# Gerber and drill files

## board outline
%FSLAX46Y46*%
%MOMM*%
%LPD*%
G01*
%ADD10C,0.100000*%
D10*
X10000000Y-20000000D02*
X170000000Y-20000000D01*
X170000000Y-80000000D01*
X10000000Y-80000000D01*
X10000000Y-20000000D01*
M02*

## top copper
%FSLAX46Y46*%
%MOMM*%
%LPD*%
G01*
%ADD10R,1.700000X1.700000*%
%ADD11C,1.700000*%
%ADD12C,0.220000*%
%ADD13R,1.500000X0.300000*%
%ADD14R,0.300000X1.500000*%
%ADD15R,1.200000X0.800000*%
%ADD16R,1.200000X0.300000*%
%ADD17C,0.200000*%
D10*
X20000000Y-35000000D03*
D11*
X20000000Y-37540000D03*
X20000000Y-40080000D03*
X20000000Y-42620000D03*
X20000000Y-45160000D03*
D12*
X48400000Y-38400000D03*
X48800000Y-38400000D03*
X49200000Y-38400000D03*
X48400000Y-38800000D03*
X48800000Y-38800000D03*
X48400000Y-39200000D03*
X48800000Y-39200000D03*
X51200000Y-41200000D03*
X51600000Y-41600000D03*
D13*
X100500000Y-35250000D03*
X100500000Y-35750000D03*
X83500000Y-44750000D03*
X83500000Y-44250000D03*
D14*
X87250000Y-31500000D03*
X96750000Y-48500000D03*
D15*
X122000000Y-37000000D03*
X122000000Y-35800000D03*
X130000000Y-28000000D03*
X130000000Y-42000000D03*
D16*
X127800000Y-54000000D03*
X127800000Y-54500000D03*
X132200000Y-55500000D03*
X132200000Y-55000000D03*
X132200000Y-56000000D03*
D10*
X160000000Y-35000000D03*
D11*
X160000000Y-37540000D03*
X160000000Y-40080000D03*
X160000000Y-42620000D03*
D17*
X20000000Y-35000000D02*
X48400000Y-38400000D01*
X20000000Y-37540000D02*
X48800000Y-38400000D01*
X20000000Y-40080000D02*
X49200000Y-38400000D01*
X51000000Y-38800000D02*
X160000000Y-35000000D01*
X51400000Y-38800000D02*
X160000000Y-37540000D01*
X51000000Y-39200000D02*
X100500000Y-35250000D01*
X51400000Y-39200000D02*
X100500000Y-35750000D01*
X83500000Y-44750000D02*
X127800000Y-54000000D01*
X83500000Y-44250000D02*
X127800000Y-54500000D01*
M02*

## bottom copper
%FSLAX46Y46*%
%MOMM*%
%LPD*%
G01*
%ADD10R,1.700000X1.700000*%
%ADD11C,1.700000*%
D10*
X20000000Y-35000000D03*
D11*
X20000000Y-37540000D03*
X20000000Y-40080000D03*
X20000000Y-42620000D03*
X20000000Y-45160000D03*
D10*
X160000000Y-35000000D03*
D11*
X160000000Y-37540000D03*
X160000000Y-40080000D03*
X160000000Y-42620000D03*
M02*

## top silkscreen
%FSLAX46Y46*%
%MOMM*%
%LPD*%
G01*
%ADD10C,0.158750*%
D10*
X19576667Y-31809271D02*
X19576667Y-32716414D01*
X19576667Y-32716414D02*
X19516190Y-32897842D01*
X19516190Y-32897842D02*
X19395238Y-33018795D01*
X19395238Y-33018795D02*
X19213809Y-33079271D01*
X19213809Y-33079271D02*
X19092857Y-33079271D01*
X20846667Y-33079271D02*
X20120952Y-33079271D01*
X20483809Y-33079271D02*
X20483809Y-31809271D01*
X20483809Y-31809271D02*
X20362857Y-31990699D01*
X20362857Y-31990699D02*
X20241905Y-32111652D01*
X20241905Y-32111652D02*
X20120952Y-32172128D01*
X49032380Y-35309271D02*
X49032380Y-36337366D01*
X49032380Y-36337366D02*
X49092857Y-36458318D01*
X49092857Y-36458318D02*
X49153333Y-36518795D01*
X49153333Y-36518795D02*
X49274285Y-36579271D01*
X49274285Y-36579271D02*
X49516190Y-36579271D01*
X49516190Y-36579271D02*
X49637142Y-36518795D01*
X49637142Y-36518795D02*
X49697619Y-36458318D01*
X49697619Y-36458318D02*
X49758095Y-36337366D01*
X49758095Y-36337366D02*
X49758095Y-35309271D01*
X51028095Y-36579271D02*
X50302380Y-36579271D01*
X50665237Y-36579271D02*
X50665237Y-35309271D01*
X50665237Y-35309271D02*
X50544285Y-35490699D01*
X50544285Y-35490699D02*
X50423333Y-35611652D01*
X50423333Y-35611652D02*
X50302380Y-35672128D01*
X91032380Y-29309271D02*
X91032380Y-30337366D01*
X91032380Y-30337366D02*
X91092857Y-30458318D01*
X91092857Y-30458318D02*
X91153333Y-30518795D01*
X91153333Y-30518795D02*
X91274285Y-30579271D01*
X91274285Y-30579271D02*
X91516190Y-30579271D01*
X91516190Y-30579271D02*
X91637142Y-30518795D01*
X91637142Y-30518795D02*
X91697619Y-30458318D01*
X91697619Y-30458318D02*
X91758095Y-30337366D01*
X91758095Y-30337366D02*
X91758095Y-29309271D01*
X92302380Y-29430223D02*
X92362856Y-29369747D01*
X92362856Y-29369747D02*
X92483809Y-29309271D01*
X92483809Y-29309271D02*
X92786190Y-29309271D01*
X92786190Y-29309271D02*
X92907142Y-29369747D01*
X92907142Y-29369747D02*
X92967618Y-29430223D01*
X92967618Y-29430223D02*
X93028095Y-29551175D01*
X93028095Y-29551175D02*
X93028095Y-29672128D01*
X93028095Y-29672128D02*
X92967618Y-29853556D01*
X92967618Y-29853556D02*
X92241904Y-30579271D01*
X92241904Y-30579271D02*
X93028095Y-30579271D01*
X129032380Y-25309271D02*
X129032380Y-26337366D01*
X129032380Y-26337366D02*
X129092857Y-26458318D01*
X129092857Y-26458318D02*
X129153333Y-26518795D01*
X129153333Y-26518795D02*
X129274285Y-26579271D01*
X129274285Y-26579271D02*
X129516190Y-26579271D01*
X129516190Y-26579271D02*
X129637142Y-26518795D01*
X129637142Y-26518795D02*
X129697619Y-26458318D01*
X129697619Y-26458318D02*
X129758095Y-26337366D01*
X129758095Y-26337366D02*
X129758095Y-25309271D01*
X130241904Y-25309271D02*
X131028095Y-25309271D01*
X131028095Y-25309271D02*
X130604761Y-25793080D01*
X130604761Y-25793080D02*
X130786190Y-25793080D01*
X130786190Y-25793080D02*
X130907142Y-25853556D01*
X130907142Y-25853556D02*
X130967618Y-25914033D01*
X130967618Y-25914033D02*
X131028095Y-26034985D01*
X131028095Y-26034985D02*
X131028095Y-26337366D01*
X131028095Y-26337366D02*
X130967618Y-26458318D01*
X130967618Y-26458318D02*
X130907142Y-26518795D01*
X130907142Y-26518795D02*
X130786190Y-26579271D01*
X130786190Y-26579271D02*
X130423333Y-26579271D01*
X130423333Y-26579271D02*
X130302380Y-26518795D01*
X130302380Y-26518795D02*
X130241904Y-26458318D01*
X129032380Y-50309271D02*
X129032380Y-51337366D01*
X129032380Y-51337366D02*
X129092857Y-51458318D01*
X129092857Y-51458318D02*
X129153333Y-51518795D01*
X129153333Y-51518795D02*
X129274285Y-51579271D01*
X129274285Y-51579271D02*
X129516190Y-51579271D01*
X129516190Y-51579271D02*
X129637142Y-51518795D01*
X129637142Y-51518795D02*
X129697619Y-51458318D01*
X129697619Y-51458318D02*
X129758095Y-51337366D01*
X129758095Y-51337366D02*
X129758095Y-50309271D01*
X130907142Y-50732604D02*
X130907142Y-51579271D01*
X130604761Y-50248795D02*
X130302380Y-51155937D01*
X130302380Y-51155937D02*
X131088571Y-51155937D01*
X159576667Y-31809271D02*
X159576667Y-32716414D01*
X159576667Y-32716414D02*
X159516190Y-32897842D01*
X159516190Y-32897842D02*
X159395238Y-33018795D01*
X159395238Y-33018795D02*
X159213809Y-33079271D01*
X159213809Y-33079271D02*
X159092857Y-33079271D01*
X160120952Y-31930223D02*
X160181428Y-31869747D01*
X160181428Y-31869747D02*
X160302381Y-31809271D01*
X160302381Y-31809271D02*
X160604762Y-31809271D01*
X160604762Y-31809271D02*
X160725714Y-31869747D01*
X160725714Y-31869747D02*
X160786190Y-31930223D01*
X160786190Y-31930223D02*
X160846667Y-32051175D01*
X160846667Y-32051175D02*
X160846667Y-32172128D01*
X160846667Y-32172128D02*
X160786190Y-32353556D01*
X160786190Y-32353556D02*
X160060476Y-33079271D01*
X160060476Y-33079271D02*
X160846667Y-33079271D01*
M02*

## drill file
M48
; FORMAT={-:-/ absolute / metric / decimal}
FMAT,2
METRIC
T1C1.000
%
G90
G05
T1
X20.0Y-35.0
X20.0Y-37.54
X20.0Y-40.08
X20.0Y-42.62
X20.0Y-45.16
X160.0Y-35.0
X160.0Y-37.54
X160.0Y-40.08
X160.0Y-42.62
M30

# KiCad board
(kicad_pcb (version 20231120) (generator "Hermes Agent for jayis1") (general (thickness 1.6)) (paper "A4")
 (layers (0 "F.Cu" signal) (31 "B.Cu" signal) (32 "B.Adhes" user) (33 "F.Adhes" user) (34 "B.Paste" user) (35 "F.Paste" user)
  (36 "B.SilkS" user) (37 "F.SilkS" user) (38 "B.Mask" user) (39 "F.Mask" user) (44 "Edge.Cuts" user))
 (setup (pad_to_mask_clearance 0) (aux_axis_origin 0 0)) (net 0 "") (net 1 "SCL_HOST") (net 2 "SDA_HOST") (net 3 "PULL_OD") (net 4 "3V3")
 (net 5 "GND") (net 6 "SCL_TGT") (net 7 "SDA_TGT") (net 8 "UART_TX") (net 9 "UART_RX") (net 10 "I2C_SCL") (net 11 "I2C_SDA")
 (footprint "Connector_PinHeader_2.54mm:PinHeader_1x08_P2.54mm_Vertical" (layer "F.Cu") (at 20 35)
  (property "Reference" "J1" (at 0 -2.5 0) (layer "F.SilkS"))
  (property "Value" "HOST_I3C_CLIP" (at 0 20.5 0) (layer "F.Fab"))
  (pad "1" thru_hole rect (at 0 0) (size 1.7 1.7) (drill 1) (layers "*.Cu" "*.Mask") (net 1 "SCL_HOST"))
  (pad "2" thru_hole circle (at 0 2.54) (size 1.7 1.7) (drill 1) (layers "*.Cu" "*.Mask") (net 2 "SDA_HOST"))
  (pad "3" thru_hole circle (at 0 5.08) (size 1.7 1.7) (drill 1) (layers "*.Cu" "*.Mask") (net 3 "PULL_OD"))
  (pad "4" thru_hole circle (at 0 7.62) (size 1.7 1.7) (drill 1) (layers "*.Cu" "*.Mask") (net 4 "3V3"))
  (pad "5" thru_hole circle (at 0 10.16) (size 1.7 1.7) (drill 1) (layers "*.Cu" "*.Mask") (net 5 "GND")))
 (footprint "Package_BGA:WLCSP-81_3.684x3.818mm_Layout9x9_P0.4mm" (layer "F.Cu") (at 50 40)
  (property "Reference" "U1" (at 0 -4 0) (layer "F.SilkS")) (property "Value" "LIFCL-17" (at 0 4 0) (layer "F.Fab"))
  (pad "A1" smd circle (at -1.6 -1.6) (size 0.22 0.22) (layers "F.Cu" "F.Paste" "F.Mask") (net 1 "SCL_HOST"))
  (pad "A2" smd circle (at -1.2 -1.6) (size 0.22 0.22) (layers "F.Cu" "F.Paste" "F.Mask") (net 2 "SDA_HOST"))
  (pad "A3" smd circle (at -0.8 -1.6) (size 0.22 0.22) (layers "F.Cu" "F.Paste" "F.Mask") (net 3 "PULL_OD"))
  (pad "B1" smd circle (at -1.6 -1.2) (size 0.22 0.22) (layers "F.Cu" "F.Paste" "F.Mask") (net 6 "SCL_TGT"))
  (pad "B2" smd circle (at -1.2 -1.2) (size 0.22 0.22) (layers "F.Cu" "F.Paste" "F.Mask") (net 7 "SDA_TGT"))
  (pad "C1" smd circle (at -1.6 -0.8) (size 0.22 0.22) (layers "F.Cu" "F.Paste" "F.Mask") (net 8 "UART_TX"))
  (pad "C2" smd circle (at -1.2 -0.8) (size 0.22 0.22) (layers "F.Cu" "F.Paste" "F.Mask") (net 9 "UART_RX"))
  (pad "H8" smd circle (at 1.2 1.2) (size 0.22 0.22) (layers "F.Cu" "F.Paste" "F.Mask") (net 4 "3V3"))
  (pad "J9" smd circle (at 1.6 1.6) (size 0.22 0.22) (layers "F.Cu" "F.Paste" "F.Mask") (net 5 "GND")))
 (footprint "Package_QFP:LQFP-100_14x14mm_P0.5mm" (layer "F.Cu") (at 92 40) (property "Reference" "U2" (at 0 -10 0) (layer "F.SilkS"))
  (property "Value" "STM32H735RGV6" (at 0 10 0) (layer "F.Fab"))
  (pad "25" smd rect (at 8.5 -4.75) (size 1.5 0.3) (layers "F.Cu" "F.Paste" "F.Mask") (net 8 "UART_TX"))
  (pad "26" smd rect (at 8.5 -4.25) (size 1.5 0.3) (layers "F.Cu" "F.Paste" "F.Mask") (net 9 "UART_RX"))
  (pad "95" smd rect (at -8.5 4.75) (size 1.5 0.3) (layers "F.Cu" "F.Paste" "F.Mask") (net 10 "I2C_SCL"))
  (pad "96" smd rect (at -8.5 4.25) (size 1.5 0.3) (layers "F.Cu" "F.Paste" "F.Mask") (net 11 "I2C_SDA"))
  (pad "13" smd rect (at -4.75 -8.5) (size 0.3 1.5) (layers "F.Cu" "F.Paste" "F.Mask") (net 4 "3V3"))
  (pad "64" smd rect (at 4.75 8.5) (size 0.3 1.5) (layers "F.Cu" "F.Paste" "F.Mask") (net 5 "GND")))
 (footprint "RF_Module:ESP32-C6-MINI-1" (layer "F.Cu") (at 130 35) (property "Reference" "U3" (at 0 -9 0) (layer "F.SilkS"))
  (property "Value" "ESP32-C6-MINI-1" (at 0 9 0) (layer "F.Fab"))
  (pad "30" smd rect (at -8 2) (size 1.2 0.8) (layers "F.Cu" "F.Paste" "F.Mask") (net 8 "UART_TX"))
  (pad "31" smd rect (at -8 0.8) (size 1.2 0.8) (layers "F.Cu" "F.Paste" "F.Mask") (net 9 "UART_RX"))
  (pad "1" smd rect (at 0 -7) (size 1.2 0.8) (layers "F.Cu" "F.Paste" "F.Mask") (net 4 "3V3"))
  (pad "15" smd rect (at 0 7) (size 1.2 0.8) (layers "F.Cu" "F.Paste" "F.Mask") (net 5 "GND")))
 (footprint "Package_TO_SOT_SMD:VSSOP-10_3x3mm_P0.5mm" (layer "F.Cu") (at 130 55) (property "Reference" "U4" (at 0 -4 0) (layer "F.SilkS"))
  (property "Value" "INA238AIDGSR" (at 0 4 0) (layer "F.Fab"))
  (pad "1" smd rect (at -2.2 -1) (size 1.2 0.3) (layers "F.Cu" "F.Paste" "F.Mask") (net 10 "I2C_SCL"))
  (pad "2" smd rect (at -2.2 -0.5) (size 1.2 0.3) (layers "F.Cu" "F.Paste" "F.Mask") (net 11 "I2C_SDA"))
  (pad "6" smd rect (at 2.2 0.5) (size 1.2 0.3) (layers "F.Cu" "F.Paste" "F.Mask") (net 4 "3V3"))
  (pad "5" smd rect (at 2.2 0) (size 1.2 0.3) (layers "F.Cu" "F.Paste" "F.Mask") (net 5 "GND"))
  (pad "8" smd rect (at 2.2 1) (size 1.2 0.3) (layers "F.Cu" "F.Paste" "F.Mask") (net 4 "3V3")))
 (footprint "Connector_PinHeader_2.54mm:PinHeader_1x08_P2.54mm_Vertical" (layer "F.Cu") (at 160 35)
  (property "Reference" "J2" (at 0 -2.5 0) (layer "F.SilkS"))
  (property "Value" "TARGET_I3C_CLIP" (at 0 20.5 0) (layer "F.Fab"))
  (pad "1" thru_hole rect (at 0 0) (size 1.7 1.7) (drill 1) (layers "*.Cu" "*.Mask") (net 6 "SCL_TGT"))
  (pad "2" thru_hole circle (at 0 2.54) (size 1.7 1.7) (drill 1) (layers "*.Cu" "*.Mask") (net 7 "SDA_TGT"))
  (pad "3" thru_hole circle (at 0 5.08) (size 1.7 1.7) (drill 1) (layers "*.Cu" "*.Mask") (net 4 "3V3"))
  (pad "4" thru_hole circle (at 0 7.62) (size 1.7 1.7) (drill 1) (layers "*.Cu" "*.Mask") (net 5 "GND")))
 (segment (start 20 35) (end 48.4 38.4) (width 0.2) (layer "F.Cu") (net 1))
 (segment (start 20 37.54) (end 48.8 38.4) (width 0.2) (layer "F.Cu") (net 2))
 (segment (start 20 40.08) (end 49.2 38.4) (width 0.2) (layer "F.Cu") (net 3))
 (segment (start 51 38.8) (end 160 35) (width 0.2) (layer "F.Cu") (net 6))
 (segment (start 51.4 38.8) (end 160 37.54) (width 0.2) (layer "F.Cu") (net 7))
 (segment (start 51 39.2) (end 100.5 35.25) (width 0.2) (layer "F.Cu") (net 8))
 (segment (start 51.4 39.2) (end 100.5 35.75) (width 0.2) (layer "F.Cu") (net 9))
 (segment (start 83.5 44.75) (end 127.8 54) (width 0.2) (layer "F.Cu") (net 10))
 (segment (start 83.5 44.25) (end 127.8 54.5) (width 0.2) (layer "F.Cu") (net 11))
 (gr_rect (start 10 20) (end 170 80) (stroke (width 0.1) (type default)) (fill none) (layer "Edge.Cuts")))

